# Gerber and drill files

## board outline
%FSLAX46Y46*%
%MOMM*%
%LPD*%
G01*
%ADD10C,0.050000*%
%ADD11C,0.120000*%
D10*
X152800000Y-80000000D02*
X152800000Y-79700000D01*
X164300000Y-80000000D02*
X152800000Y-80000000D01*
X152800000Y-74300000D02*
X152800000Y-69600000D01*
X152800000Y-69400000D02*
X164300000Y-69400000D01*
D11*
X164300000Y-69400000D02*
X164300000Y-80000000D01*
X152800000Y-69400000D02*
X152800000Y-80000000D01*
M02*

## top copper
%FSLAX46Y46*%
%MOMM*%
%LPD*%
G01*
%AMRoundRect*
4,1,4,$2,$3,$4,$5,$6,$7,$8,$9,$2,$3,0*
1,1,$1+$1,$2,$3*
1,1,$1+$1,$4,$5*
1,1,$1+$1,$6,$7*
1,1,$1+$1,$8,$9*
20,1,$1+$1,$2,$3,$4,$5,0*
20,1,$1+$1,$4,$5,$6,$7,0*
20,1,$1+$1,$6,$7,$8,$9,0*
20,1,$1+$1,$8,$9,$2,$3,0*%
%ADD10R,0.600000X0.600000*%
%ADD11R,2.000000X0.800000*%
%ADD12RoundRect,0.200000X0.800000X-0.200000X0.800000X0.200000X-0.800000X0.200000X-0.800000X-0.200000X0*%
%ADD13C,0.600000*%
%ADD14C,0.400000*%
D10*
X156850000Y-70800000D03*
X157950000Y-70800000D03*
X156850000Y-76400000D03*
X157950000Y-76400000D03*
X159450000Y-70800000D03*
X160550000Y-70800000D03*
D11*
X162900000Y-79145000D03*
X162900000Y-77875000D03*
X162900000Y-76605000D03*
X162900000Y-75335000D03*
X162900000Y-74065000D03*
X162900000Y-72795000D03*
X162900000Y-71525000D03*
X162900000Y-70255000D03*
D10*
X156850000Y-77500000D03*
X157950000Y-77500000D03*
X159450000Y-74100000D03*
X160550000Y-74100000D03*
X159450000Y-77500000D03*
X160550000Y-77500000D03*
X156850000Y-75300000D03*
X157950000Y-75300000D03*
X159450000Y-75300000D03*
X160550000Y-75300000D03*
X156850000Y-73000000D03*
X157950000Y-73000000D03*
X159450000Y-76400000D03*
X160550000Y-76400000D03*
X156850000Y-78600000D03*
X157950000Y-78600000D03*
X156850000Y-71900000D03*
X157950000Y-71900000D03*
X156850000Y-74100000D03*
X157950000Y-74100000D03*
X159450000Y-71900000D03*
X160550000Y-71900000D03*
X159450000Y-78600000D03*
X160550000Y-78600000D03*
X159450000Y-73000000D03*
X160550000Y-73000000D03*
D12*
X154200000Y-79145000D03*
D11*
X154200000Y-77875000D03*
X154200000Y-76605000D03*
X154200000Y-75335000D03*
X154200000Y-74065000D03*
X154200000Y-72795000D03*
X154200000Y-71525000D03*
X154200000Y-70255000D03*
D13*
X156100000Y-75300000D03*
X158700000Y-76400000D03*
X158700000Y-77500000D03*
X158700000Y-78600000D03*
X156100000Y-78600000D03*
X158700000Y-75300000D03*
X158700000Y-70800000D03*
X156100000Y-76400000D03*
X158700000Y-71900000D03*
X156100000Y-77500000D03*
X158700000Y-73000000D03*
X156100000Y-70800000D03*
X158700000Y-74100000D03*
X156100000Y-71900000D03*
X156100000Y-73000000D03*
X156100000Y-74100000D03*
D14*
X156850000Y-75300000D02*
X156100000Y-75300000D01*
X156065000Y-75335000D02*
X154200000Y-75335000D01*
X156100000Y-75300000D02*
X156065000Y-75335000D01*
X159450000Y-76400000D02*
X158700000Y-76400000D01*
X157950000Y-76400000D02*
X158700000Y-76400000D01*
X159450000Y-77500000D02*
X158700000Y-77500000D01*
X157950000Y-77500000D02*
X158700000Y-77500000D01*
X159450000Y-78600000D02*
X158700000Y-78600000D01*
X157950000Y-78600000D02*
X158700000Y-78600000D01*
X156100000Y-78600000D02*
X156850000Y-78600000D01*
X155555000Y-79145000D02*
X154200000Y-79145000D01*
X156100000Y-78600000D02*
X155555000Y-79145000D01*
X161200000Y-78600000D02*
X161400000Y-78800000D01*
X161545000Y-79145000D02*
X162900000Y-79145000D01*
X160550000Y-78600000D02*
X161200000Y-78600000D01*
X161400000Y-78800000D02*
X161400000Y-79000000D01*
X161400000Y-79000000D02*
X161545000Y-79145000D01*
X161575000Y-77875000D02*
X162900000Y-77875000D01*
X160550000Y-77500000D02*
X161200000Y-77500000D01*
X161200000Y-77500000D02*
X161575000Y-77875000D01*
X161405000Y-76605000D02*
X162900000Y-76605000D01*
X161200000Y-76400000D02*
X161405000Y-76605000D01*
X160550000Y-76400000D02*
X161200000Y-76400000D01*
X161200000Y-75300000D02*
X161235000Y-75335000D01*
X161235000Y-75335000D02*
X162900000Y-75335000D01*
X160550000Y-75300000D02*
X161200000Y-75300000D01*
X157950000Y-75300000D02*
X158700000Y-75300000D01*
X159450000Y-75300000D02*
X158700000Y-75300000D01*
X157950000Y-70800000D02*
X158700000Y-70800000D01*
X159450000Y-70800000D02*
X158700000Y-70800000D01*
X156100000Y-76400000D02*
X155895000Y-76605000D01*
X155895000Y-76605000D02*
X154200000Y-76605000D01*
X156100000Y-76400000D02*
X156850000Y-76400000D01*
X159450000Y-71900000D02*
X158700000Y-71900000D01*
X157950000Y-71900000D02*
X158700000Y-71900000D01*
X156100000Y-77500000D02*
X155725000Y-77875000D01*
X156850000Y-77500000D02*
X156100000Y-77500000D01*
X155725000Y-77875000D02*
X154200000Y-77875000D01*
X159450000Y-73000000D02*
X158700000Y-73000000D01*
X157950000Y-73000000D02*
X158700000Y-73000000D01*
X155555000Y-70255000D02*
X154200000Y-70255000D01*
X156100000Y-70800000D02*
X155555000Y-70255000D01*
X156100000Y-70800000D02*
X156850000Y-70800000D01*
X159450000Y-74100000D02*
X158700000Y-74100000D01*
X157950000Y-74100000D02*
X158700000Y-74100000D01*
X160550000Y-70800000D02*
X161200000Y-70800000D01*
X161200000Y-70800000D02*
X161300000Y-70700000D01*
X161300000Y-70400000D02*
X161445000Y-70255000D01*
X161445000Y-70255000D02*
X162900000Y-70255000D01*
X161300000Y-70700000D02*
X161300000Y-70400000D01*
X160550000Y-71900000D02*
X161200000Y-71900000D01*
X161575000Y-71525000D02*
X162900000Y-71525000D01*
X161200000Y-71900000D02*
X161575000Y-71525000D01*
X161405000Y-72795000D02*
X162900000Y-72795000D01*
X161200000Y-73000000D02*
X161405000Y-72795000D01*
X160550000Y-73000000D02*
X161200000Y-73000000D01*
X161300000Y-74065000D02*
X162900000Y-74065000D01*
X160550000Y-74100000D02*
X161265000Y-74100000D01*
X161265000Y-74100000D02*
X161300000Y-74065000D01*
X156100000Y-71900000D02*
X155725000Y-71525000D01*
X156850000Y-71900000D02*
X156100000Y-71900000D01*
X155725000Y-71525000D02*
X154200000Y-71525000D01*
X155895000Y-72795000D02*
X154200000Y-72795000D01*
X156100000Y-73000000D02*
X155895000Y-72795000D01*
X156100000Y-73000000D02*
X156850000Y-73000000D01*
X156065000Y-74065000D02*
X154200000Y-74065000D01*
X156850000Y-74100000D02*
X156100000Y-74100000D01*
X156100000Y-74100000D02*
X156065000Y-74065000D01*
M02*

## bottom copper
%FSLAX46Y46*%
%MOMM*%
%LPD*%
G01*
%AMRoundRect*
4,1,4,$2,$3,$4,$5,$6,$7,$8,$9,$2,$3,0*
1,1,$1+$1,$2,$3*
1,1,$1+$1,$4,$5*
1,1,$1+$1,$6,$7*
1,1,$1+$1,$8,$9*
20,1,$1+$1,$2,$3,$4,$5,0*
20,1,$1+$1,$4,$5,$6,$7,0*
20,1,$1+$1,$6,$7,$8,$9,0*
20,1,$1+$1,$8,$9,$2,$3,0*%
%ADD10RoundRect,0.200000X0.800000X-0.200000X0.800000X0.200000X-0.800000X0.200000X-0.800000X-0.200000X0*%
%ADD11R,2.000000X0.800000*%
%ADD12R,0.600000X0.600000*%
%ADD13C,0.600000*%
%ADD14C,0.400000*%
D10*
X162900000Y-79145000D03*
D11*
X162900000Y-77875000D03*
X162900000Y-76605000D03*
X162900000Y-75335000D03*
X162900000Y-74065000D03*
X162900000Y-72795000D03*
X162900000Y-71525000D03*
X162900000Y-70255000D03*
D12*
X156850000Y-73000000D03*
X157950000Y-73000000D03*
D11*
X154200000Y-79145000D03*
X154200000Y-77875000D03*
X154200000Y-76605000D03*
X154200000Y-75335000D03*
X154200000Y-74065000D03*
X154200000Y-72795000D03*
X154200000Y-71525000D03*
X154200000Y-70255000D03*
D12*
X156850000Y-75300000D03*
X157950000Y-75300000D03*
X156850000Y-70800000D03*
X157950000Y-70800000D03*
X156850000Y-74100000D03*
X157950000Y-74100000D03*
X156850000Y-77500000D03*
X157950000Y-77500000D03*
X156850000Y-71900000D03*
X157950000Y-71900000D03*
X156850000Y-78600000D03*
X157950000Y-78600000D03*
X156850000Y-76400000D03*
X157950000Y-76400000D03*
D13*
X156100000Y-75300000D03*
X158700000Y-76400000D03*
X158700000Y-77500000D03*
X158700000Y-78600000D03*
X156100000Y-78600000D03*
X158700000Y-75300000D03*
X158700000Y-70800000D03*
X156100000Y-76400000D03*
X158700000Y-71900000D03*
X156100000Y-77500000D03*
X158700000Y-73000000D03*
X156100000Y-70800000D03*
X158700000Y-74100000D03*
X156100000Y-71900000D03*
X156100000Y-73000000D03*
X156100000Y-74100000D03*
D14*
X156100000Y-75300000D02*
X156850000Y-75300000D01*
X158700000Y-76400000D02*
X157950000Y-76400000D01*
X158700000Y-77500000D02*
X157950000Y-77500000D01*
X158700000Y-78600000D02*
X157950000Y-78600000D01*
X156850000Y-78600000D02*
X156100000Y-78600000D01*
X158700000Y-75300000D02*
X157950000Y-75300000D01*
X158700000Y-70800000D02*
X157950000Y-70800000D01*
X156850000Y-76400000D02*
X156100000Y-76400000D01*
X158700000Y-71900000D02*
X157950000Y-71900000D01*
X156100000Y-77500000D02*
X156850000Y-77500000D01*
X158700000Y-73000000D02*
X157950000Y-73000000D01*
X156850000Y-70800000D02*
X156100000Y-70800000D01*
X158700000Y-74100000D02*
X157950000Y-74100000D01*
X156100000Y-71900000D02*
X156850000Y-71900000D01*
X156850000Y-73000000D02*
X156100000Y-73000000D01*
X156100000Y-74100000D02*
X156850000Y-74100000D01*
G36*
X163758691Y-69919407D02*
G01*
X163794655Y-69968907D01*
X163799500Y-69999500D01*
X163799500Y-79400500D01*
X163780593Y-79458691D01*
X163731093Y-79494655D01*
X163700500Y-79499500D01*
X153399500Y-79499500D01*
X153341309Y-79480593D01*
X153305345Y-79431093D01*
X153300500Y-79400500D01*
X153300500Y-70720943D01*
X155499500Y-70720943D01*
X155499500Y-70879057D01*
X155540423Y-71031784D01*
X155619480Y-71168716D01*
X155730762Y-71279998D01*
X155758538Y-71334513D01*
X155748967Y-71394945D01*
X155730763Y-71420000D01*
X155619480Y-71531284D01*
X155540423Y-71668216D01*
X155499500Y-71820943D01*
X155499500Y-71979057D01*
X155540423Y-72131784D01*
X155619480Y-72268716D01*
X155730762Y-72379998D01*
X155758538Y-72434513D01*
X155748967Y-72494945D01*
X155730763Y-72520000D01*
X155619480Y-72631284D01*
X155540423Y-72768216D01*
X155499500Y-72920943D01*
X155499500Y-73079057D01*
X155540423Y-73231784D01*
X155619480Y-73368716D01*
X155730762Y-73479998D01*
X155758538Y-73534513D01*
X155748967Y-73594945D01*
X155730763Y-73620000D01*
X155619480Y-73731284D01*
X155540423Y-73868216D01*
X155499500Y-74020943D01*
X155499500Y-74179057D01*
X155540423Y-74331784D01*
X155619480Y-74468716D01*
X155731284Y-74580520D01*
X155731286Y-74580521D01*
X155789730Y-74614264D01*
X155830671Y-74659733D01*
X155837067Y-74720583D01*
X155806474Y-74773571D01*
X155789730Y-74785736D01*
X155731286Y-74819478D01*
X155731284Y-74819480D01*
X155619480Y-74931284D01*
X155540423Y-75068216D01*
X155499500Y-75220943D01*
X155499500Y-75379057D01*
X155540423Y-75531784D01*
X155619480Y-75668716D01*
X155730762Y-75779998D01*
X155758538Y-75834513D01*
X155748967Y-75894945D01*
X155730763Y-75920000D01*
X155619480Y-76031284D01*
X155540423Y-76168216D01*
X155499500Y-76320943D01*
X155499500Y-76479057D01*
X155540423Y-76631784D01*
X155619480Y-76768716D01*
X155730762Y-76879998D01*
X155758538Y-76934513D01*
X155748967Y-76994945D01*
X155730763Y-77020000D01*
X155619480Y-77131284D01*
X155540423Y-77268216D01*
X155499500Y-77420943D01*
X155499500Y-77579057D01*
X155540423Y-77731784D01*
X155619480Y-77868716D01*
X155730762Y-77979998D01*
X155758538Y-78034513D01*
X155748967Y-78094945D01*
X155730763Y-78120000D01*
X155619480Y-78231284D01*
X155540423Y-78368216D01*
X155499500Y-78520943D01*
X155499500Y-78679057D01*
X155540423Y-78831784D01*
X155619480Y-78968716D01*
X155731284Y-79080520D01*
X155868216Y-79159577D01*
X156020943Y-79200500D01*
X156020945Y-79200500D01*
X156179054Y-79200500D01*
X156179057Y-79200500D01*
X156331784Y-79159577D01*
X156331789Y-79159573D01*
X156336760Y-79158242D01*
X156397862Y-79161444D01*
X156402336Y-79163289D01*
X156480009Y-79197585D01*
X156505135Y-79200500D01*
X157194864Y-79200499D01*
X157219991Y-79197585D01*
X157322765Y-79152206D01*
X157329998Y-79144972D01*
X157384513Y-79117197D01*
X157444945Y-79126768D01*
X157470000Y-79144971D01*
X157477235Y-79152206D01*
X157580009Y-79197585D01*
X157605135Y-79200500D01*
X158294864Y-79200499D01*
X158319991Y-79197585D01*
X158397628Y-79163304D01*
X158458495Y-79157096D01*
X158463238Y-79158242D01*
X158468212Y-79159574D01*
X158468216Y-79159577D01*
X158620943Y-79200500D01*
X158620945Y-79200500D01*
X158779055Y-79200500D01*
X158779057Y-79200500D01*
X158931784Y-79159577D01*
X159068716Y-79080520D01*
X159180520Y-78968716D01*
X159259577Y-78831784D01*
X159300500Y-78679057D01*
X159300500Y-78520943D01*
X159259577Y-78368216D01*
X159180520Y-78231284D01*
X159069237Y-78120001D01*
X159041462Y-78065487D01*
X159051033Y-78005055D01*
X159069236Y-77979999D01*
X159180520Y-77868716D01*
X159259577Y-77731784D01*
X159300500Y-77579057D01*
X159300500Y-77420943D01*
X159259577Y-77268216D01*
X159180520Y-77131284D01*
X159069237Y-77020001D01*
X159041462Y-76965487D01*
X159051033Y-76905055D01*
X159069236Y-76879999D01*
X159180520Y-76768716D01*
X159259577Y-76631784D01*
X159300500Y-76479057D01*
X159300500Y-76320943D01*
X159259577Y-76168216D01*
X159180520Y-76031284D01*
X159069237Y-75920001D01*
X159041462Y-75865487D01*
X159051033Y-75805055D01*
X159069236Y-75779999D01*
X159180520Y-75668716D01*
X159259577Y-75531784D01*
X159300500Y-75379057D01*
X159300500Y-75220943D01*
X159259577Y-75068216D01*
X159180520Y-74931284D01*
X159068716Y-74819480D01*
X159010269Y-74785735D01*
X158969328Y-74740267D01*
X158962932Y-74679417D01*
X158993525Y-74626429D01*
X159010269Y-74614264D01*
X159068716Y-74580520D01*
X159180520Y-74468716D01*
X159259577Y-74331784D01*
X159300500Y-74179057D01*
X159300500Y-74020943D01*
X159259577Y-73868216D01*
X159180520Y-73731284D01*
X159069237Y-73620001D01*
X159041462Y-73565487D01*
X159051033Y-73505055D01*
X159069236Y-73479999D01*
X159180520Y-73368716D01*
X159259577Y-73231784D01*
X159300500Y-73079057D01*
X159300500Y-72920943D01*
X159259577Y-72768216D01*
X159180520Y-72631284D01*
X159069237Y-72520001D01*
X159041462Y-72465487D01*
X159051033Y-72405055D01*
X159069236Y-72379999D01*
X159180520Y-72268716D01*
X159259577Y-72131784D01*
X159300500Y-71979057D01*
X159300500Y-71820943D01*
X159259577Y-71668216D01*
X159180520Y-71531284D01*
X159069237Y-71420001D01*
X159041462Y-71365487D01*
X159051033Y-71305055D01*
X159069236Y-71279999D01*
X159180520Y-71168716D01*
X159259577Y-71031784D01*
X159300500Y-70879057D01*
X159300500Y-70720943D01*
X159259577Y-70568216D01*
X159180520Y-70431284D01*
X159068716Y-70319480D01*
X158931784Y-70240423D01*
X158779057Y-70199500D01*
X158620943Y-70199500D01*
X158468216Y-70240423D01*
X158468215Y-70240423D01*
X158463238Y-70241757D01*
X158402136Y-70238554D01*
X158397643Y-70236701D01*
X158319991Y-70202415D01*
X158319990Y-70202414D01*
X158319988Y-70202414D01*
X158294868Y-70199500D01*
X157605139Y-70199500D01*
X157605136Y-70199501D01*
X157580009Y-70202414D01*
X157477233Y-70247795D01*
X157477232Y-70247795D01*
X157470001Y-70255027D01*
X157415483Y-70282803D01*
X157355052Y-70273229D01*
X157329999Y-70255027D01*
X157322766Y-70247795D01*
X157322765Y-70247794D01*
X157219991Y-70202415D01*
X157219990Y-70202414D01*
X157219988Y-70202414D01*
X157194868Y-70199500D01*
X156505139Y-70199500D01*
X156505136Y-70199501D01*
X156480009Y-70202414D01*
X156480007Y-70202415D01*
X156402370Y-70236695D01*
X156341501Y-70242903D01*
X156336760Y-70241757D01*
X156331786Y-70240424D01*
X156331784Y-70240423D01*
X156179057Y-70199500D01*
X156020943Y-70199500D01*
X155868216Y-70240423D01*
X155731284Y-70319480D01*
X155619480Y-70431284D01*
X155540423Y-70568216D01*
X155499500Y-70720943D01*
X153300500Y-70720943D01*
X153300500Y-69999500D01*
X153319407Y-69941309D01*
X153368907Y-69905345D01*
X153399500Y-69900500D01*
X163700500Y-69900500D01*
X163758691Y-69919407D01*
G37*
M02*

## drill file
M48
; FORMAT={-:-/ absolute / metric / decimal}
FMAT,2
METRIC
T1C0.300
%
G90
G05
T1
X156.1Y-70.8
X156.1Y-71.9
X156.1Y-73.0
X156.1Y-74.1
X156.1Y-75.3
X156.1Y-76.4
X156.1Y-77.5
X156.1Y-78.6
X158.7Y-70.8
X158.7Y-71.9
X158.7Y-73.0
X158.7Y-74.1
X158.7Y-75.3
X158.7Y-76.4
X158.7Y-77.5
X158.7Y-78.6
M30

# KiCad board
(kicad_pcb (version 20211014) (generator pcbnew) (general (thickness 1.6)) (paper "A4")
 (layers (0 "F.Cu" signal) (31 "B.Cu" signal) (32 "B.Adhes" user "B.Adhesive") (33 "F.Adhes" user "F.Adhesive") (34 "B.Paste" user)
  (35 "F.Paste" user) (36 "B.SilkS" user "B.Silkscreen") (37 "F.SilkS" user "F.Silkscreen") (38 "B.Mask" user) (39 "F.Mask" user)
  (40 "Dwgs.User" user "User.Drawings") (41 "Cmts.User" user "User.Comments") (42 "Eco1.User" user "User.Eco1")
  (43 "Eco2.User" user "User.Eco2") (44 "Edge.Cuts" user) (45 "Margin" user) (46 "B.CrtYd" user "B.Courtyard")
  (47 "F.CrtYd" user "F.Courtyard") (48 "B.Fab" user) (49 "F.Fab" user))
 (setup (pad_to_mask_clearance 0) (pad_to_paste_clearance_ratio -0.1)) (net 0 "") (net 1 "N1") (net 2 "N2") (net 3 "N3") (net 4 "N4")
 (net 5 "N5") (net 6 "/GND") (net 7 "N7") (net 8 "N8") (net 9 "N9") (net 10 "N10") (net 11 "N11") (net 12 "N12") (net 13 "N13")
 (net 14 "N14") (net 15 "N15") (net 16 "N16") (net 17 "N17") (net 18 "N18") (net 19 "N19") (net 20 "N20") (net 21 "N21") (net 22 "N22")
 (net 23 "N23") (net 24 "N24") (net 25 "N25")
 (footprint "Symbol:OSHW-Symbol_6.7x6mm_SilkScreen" (layer "F.Cu") (at 147 76.2)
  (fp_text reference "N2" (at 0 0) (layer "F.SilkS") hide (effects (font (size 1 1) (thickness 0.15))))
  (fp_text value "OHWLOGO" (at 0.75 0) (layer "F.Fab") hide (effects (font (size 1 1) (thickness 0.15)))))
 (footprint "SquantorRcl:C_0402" (layer "F.Cu") (at 157.4 70.8)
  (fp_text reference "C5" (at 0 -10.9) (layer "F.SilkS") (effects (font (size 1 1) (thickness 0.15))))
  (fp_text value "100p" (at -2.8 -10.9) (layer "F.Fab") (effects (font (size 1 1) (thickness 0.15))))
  (pad "1" smd rect (at -0.55 0) (size 0.6 0.6) (layers "F.Cu" "F.Paste" "F.Mask") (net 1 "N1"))
  (pad "2" smd rect (at 0.55 0) (size 0.6 0.6) (layers "F.Cu" "F.Paste" "F.Mask") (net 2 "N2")))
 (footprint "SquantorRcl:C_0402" (layer "F.Cu") (at 157.4 76.4)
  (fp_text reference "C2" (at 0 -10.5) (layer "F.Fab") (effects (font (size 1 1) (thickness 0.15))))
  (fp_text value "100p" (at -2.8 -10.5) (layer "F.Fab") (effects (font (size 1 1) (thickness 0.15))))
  (pad "1" smd rect (at -0.55 0) (size 0.6 0.6) (layers "F.Cu" "F.Paste" "F.Mask") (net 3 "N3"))
  (pad "2" smd rect (at 0.55 0) (size 0.6 0.6) (layers "F.Cu" "F.Paste" "F.Mask") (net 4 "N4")))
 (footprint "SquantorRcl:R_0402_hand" (layer "F.Cu") (at 160 70.8)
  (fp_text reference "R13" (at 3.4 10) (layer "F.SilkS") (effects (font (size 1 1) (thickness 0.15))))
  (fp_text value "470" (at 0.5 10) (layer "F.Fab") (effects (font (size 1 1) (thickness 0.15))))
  (pad "1" smd rect (at -0.55 0) (size 0.6 0.6) (layers "F.Cu" "F.Paste" "F.Mask") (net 2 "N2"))
  (pad "2" smd rect (at 0.55 0) (size 0.6 0.6) (layers "F.Cu" "F.Paste" "F.Mask") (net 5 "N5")))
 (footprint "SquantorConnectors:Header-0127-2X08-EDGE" (layer "F.Cu") (at 161.8 74.7 90)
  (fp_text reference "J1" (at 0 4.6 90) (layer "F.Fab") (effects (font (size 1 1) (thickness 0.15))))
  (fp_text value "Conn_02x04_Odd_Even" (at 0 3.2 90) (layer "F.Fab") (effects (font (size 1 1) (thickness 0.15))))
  (fp_line (start 5.3 2.5) (end -5.3 2.5) (layer "Edge.Cuts") (width 0.12))
  (pad "1" smd roundrect (at -4.445 1.1 90) (size 0.8 2) (layers "B.Cu" "B.Paste" "B.Mask") (roundrect_rratio 0.25) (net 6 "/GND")
   (zone_connect 2))
  (pad "2" smd rect (at -4.445 1.1 90) (size 0.8 2) (layers "F.Cu" "F.Paste" "F.Mask") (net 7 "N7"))
  (pad "3" smd rect (at -3.175 1.1 90) (size 0.8 2) (layers "B.Cu" "B.Paste" "B.Mask") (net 6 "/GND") (zone_connect 2))
  (pad "4" smd rect (at -3.175 1.1 90) (size 0.8 2) (layers "F.Cu" "F.Paste" "F.Mask") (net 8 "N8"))
  (pad "5" smd rect (at -1.905 1.1 90) (size 0.8 2) (layers "B.Cu" "B.Paste" "B.Mask") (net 6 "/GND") (zone_connect 2))
  (pad "6" smd rect (at -1.905 1.1 90) (size 0.8 2) (layers "F.Cu" "F.Paste" "F.Mask") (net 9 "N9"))
  (pad "7" smd rect (at -0.635 1.1 90) (size 0.8 2) (layers "B.Cu" "B.Paste" "B.Mask") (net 6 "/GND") (zone_connect 2))
  (pad "8" smd rect (at -0.635 1.1 90) (size 0.8 2) (layers "F.Cu" "F.Paste" "F.Mask") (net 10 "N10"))
  (pad "9" smd rect (at 0.635 1.1 90) (size 0.8 2) (layers "B.Cu" "B.Paste" "B.Mask") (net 6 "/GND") (zone_connect 2))
  (pad "10" smd rect (at 0.635 1.1 90) (size 0.8 2) (layers "F.Cu" "F.Paste" "F.Mask") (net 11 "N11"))
  (pad "11" smd rect (at 1.905 1.1 90) (size 0.8 2) (layers "B.Cu" "B.Paste" "B.Mask") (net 6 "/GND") (zone_connect 2))
  (pad "12" smd rect (at 1.905 1.1 90) (size 0.8 2) (layers "F.Cu" "F.Paste" "F.Mask") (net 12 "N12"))
  (pad "13" smd rect (at 3.175 1.1 90) (size 0.8 2) (layers "B.Cu" "B.Paste" "B.Mask") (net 6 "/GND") (zone_connect 2))
  (pad "14" smd rect (at 3.175 1.1 90) (size 0.8 2) (layers "F.Cu" "F.Paste" "F.Mask") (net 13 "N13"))
  (pad "15" smd rect (at 4.445 1.1 90) (size 0.8 2) (layers "B.Cu" "B.Paste" "B.Mask") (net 6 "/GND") (zone_connect 2))
  (pad "16" smd rect (at 4.445 1.1 90) (size 0.8 2) (layers "F.Cu" "F.Paste" "F.Mask") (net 5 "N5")))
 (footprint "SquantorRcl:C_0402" (layer "F.Cu") (at 157.4 77.5)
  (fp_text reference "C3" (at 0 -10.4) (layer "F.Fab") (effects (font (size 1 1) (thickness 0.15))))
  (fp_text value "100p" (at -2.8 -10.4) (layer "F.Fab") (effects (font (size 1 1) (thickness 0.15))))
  (pad "1" smd rect (at -0.55 0) (size 0.6 0.6) (layers "F.Cu" "F.Paste" "F.Mask") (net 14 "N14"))
  (pad "2" smd rect (at 0.55 0) (size 0.6 0.6) (layers "F.Cu" "F.Paste" "F.Mask") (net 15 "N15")))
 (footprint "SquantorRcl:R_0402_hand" (layer "F.Cu") (at 160 74.1)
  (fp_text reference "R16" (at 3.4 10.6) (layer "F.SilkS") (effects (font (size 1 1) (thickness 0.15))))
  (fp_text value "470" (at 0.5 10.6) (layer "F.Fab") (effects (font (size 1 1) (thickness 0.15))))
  (pad "1" smd rect (at -0.55 0) (size 0.6 0.6) (layers "F.Cu" "F.Paste" "F.Mask") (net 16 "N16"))
  (pad "2" smd rect (at 0.55 0) (size 0.6 0.6) (layers "F.Cu" "F.Paste" "F.Mask") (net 11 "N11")))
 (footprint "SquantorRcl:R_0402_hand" (layer "F.Cu") (at 160 77.5)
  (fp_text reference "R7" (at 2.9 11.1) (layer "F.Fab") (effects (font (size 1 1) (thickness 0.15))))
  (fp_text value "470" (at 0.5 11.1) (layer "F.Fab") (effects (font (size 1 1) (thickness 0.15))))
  (pad "1" smd rect (at -0.55 0) (size 0.6 0.6) (layers "F.Cu" "F.Paste" "F.Mask") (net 15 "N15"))
  (pad "2" smd rect (at 0.55 0) (size 0.6 0.6) (layers "F.Cu" "F.Paste" "F.Mask") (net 8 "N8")))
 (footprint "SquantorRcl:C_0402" (layer "F.Cu") (at 157.4 75.3)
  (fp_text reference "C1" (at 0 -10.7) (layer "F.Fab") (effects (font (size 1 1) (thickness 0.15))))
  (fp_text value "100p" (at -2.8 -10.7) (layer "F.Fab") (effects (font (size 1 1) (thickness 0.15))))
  (pad "1" smd rect (at -0.55 0) (size 0.6 0.6) (layers "F.Cu" "F.Paste" "F.Mask") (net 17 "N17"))
  (pad "2" smd rect (at 0.55 0) (size 0.6 0.6) (layers "F.Cu" "F.Paste" "F.Mask") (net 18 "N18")))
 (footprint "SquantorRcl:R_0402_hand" (layer "F.Cu") (at 160 75.3)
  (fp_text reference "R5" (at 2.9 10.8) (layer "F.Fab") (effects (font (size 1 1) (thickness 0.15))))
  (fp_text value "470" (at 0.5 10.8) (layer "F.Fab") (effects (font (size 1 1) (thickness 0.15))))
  (pad "1" smd rect (at -0.55 0) (size 0.6 0.6) (layers "F.Cu" "F.Paste" "F.Mask") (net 18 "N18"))
  (pad "2" smd rect (at 0.55 0) (size 0.6 0.6) (layers "F.Cu" "F.Paste" "F.Mask") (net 10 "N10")))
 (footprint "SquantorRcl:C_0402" (layer "F.Cu") (at 157.4 73)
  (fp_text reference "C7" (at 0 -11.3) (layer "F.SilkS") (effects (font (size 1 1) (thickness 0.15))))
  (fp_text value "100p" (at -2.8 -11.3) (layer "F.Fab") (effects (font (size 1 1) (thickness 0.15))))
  (pad "1" smd rect (at -0.55 0) (size 0.6 0.6) (layers "F.Cu" "F.Paste" "F.Mask") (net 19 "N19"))
  (pad "2" smd rect (at 0.55 0) (size 0.6 0.6) (layers "F.Cu" "F.Paste" "F.Mask") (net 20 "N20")))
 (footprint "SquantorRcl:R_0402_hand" (layer "F.Cu") (at 160 76.4)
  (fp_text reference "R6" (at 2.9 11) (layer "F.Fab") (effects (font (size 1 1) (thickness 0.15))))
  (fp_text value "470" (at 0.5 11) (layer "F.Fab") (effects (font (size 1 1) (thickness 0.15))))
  (pad "1" smd rect (at -0.55 0) (size 0.6 0.6) (layers "F.Cu" "F.Paste" "F.Mask") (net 4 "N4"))
  (pad "2" smd rect (at 0.55 0) (size 0.6 0.6) (layers "F.Cu" "F.Paste" "F.Mask") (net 9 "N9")))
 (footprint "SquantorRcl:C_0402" (layer "F.Cu") (at 157.4 78.6)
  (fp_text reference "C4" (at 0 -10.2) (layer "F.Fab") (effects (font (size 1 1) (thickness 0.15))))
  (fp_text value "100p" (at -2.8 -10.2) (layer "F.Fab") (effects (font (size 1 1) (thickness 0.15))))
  (pad "1" smd rect (at -0.55 0) (size 0.6 0.6) (layers "F.Cu" "F.Paste" "F.Mask") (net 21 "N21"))
  (pad "2" smd rect (at 0.55 0) (size 0.6 0.6) (layers "F.Cu" "F.Paste" "F.Mask") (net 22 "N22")))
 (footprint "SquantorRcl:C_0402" (layer "F.Cu") (at 157.4 71.9)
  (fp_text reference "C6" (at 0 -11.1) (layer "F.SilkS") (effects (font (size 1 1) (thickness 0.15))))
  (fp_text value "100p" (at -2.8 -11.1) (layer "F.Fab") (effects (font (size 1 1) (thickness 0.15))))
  (pad "1" smd rect (at -0.55 0) (size 0.6 0.6) (layers "F.Cu" "F.Paste" "F.Mask") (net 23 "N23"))
  (pad "2" smd rect (at 0.55 0) (size 0.6 0.6) (layers "F.Cu" "F.Paste" "F.Mask") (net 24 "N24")))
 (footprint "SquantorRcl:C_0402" (layer "F.Cu") (at 157.4 74.1)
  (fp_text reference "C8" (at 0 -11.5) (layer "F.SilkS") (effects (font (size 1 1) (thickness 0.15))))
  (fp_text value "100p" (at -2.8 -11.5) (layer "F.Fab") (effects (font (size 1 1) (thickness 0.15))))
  (pad "1" smd rect (at -0.55 0) (size 0.6 0.6) (layers "F.Cu" "F.Paste" "F.Mask") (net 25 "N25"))
  (pad "2" smd rect (at 0.55 0) (size 0.6 0.6) (layers "F.Cu" "F.Paste" "F.Mask") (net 16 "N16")))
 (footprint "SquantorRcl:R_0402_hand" (layer "F.Cu") (at 160 71.9)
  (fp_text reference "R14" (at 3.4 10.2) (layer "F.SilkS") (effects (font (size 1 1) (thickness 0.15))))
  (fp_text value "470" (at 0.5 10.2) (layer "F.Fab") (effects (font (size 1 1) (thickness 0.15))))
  (pad "1" smd rect (at -0.55 0) (size 0.6 0.6) (layers "F.Cu" "F.Paste" "F.Mask") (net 24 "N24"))
  (pad "2" smd rect (at 0.55 0) (size 0.6 0.6) (layers "F.Cu" "F.Paste" "F.Mask") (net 13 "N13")))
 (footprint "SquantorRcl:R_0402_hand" (layer "F.Cu") (at 160 78.6)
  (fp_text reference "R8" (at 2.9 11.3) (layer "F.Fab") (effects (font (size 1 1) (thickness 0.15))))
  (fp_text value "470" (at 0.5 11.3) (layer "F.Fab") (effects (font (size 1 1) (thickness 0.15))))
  (pad "1" smd rect (at -0.55 0) (size 0.6 0.6) (layers "F.Cu" "F.Paste" "F.Mask") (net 22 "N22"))
  (pad "2" smd rect (at 0.55 0) (size 0.6 0.6) (layers "F.Cu" "F.Paste" "F.Mask") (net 7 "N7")))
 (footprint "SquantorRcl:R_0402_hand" (layer "F.Cu") (at 160 73)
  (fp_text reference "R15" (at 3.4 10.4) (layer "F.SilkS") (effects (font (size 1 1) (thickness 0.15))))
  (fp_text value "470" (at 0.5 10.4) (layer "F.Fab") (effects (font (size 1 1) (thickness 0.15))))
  (pad "1" smd rect (at -0.55 0) (size 0.6 0.6) (layers "F.Cu" "F.Paste" "F.Mask") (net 20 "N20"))
  (pad "2" smd rect (at 0.55 0) (size 0.6 0.6) (layers "F.Cu" "F.Paste" "F.Mask") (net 12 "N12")))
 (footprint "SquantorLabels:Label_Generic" (layer "B.Cu") (at 159.7875 74.4 -90)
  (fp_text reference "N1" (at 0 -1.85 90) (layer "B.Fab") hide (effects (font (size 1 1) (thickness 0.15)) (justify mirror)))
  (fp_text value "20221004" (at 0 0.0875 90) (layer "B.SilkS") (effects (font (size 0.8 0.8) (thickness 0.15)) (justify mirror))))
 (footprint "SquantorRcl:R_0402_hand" (layer "B.Cu") (at 157.4 73)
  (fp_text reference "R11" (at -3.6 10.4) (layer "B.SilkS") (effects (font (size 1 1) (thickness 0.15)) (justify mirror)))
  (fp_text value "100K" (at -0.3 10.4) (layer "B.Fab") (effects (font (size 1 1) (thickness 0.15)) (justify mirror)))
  (pad "1" smd rect (at -0.55 0) (size 0.6 0.6) (layers "B.Cu" "B.Paste" "B.Mask") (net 19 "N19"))
  (pad "2" smd rect (at 0.55 0) (size 0.6 0.6) (layers "B.Cu" "B.Paste" "B.Mask") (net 20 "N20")))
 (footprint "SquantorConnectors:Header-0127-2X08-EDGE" (layer "B.Cu") (at 155.3 74.7 90)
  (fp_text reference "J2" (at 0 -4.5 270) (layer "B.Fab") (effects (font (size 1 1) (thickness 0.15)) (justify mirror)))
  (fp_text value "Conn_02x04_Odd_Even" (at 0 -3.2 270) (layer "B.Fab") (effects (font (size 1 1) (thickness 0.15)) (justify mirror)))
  (fp_line (start 5.3 -2.5) (end -5.3 -2.5) (layer "Edge.Cuts") (width 0.12))
  (pad "1" smd roundrect (at -4.445 -1.1 90) (size 0.8 2) (layers "F.Cu" "F.Paste" "F.Mask") (roundrect_rratio 0.25) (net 21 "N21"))
  (pad "2" smd rect (at -4.445 -1.1 90) (size 0.8 2) (layers "B.Cu" "B.Paste" "B.Mask") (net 6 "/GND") (zone_connect 2))
  (pad "3" smd rect (at -3.175 -1.1 90) (size 0.8 2) (layers "F.Cu" "F.Paste" "F.Mask") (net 14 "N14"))
  (pad "4" smd rect (at -3.175 -1.1 90) (size 0.8 2) (layers "B.Cu" "B.Paste" "B.Mask") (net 6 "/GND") (zone_connect 2))
  (pad "5" smd rect (at -1.905 -1.1 90) (size 0.8 2) (layers "F.Cu" "F.Paste" "F.Mask") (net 3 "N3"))
  (pad "6" smd rect (at -1.905 -1.1 90) (size 0.8 2) (layers "B.Cu" "B.Paste" "B.Mask") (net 6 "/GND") (zone_connect 2))
  (pad "7" smd rect (at -0.635 -1.1 90) (size 0.8 2) (layers "F.Cu" "F.Paste" "F.Mask") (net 17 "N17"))
  (pad "8" smd rect (at -0.635 -1.1 90) (size 0.8 2) (layers "B.Cu" "B.Paste" "B.Mask") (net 6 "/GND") (zone_connect 2))
  (pad "9" smd rect (at 0.635 -1.1 90) (size 0.8 2) (layers "F.Cu" "F.Paste" "F.Mask") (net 25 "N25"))
  (pad "10" smd rect (at 0.635 -1.1 90) (size 0.8 2) (layers "B.Cu" "B.Paste" "B.Mask") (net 6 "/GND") (zone_connect 2))
  (pad "11" smd rect (at 1.905 -1.1 90) (size 0.8 2) (layers "F.Cu" "F.Paste" "F.Mask") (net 19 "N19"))
  (pad "12" smd rect (at 1.905 -1.1 90) (size 0.8 2) (layers "B.Cu" "B.Paste" "B.Mask") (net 6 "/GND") (zone_connect 2))
  (pad "13" smd rect (at 3.175 -1.1 90) (size 0.8 2) (layers "F.Cu" "F.Paste" "F.Mask") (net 23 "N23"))
  (pad "14" smd rect (at 3.175 -1.1 90) (size 0.8 2) (layers "B.Cu" "B.Paste" "B.Mask") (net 6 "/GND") (zone_connect 2))
  (pad "15" smd rect (at 4.445 -1.1 90) (size 0.8 2) (layers "F.Cu" "F.Paste" "F.Mask") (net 1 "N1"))
  (pad "16" smd rect (at 4.445 -1.1 90) (size 0.8 2) (layers "B.Cu" "B.Paste" "B.Mask") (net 6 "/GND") (zone_connect 2)))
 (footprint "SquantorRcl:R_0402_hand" (layer "B.Cu") (at 157.4 75.3)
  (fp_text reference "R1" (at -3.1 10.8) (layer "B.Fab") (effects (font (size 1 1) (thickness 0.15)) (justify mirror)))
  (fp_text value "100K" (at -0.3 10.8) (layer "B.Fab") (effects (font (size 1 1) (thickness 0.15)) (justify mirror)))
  (pad "1" smd rect (at -0.55 0) (size 0.6 0.6) (layers "B.Cu" "B.Paste" "B.Mask") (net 17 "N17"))
  (pad "2" smd rect (at 0.55 0) (size 0.6 0.6) (layers "B.Cu" "B.Paste" "B.Mask") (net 18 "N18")))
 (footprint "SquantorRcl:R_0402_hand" (layer "B.Cu") (at 157.4 70.8)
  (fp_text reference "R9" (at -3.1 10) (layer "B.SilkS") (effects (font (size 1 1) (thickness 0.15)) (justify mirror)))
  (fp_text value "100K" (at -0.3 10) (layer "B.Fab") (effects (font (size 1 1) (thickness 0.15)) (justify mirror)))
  (pad "1" smd rect (at -0.55 0) (size 0.6 0.6) (layers "B.Cu" "B.Paste" "B.Mask") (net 1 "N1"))
  (pad "2" smd rect (at 0.55 0) (size 0.6 0.6) (layers "B.Cu" "B.Paste" "B.Mask") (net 2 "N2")))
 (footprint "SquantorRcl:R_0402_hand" (layer "B.Cu") (at 157.4 74.1)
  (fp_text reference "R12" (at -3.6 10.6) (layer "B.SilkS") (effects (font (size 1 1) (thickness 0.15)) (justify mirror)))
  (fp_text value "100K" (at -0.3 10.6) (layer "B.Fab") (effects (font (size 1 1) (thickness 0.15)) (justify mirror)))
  (pad "1" smd rect (at -0.55 0) (size 0.6 0.6) (layers "B.Cu" "B.Paste" "B.Mask") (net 25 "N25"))
  (pad "2" smd rect (at 0.55 0) (size 0.6 0.6) (layers "B.Cu" "B.Paste" "B.Mask") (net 16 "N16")))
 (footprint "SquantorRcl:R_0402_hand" (layer "B.Cu") (at 157.4 77.5)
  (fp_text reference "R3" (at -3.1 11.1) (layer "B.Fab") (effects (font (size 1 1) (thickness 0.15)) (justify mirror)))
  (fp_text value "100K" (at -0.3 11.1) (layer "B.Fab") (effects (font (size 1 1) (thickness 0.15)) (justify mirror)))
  (pad "1" smd rect (at -0.55 0) (size 0.6 0.6) (layers "B.Cu" "B.Paste" "B.Mask") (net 14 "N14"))
  (pad "2" smd rect (at 0.55 0) (size 0.6 0.6) (layers "B.Cu" "B.Paste" "B.Mask") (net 15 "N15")))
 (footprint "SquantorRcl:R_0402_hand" (layer "B.Cu") (at 157.4 71.9)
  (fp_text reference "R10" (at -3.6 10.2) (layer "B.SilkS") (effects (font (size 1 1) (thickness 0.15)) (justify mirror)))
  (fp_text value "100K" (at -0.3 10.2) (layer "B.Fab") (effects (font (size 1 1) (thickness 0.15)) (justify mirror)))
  (pad "1" smd rect (at -0.55 0) (size 0.6 0.6) (layers "B.Cu" "B.Paste" "B.Mask") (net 23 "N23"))
  (pad "2" smd rect (at 0.55 0) (size 0.6 0.6) (layers "B.Cu" "B.Paste" "B.Mask") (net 24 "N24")))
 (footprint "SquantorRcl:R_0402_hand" (layer "B.Cu") (at 157.4 78.6)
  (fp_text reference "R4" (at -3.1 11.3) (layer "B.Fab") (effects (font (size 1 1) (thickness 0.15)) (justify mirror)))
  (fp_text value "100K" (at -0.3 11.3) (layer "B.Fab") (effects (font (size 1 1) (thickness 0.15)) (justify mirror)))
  (pad "1" smd rect (at -0.55 0) (size 0.6 0.6) (layers "B.Cu" "B.Paste" "B.Mask") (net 21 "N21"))
  (pad "2" smd rect (at 0.55 0) (size 0.6 0.6) (layers "B.Cu" "B.Paste" "B.Mask") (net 22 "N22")))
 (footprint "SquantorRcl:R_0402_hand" (layer "B.Cu") (at 157.4 76.4)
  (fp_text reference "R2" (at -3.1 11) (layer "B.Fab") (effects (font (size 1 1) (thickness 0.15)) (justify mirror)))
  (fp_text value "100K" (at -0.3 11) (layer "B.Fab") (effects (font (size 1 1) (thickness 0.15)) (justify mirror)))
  (pad "1" smd rect (at -0.55 0) (size 0.6 0.6) (layers "B.Cu" "B.Paste" "B.Mask") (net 3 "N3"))
  (pad "2" smd rect (at 0.55 0) (size 0.6 0.6) (layers "B.Cu" "B.Paste" "B.Mask") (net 4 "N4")))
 (gr_line (start 152.8 80) (end 152.8 79.7) (layer "Edge.Cuts") (width 0.05))
 (gr_line (start 164.3 80) (end 152.8 80) (layer "Edge.Cuts") (width 0.05))
 (gr_line (start 152.8 74.3) (end 152.8 69.6) (layer "Edge.Cuts") (width 0.05))
 (gr_line (start 152.8 69.4) (end 164.3 69.4) (layer "Edge.Cuts") (width 0.05))
 (segment (start 156.85 75.3) (end 156.1 75.3) (width 0.4) (layer "F.Cu") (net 17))
 (segment (start 156.065 75.335) (end 154.2 75.335) (width 0.4) (layer "F.Cu") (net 17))
 (segment (start 156.1 75.3) (end 156.065 75.335) (width 0.4) (layer "F.Cu") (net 17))
 (via (at 156.1 75.3) (size 0.6) (drill 0.3) (layers "F.Cu" "B.Cu") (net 17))
 (segment (start 156.1 75.3) (end 156.85 75.3) (width 0.4) (layer "B.Cu") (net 17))
 (segment (start 159.45 76.4) (end 158.7 76.4) (width 0.4) (layer "F.Cu") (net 4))
 (segment (start 157.95 76.4) (end 158.7 76.4) (width 0.4) (layer "F.Cu") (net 4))
 (via (at 158.7 76.4) (size 0.6) (drill 0.3) (layers "F.Cu" "B.Cu") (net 4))
 (segment (start 158.7 76.4) (end 157.95 76.4) (width 0.4) (layer "B.Cu") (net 4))
 (segment (start 159.45 77.5) (end 158.7 77.5) (width 0.4) (layer "F.Cu") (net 15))
 (segment (start 157.95 77.5) (end 158.7 77.5) (width 0.4) (layer "F.Cu") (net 15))
 (via (at 158.7 77.5) (size 0.6) (drill 0.3) (layers "F.Cu" "B.Cu") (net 15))
 (segment (start 158.7 77.5) (end 157.95 77.5) (width 0.4) (layer "B.Cu") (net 15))
 (segment (start 159.45 78.6) (end 158.7 78.6) (width 0.4) (layer "F.Cu") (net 22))
 (segment (start 157.95 78.6) (end 158.7 78.6) (width 0.4) (layer "F.Cu") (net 22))
 (via (at 158.7 78.6) (size 0.6) (drill 0.3) (layers "F.Cu" "B.Cu") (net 22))
 (segment (start 158.7 78.6) (end 157.95 78.6) (width 0.4) (layer "B.Cu") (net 22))
 (segment (start 156.1 78.6) (end 156.85 78.6) (width 0.4) (layer "F.Cu") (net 21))
 (segment (start 155.555 79.145) (end 154.2 79.145) (width 0.4) (layer "F.Cu") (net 21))
 (segment (start 156.1 78.6) (end 155.555 79.145) (width 0.4) (layer "F.Cu") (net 21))
 (via (at 156.1 78.6) (size 0.6) (drill 0.3) (layers "F.Cu" "B.Cu") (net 21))
 (segment (start 156.85 78.6) (end 156.1 78.6) (width 0.4) (layer "B.Cu") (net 21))
 (segment (start 161.2 78.6) (end 161.4 78.8) (width 0.4) (layer "F.Cu") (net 7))
 (segment (start 161.545 79.145) (end 162.9 79.145) (width 0.4) (layer "F.Cu") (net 7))
 (segment (start 160.55 78.6) (end 161.2 78.6) (width 0.4) (layer "F.Cu") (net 7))
 (segment (start 161.4 78.8) (end 161.4 79) (width 0.4) (layer "F.Cu") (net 7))
 (segment (start 161.4 79) (end 161.545 79.145) (width 0.4) (layer "F.Cu") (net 7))
 (segment (start 161.575 77.875) (end 162.9 77.875) (width 0.4) (layer "F.Cu") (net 8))
 (segment (start 160.55 77.5) (end 161.2 77.5) (width 0.4) (layer "F.Cu") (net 8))
 (segment (start 161.2 77.5) (end 161.575 77.875) (width 0.4) (layer "F.Cu") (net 8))
 (segment (start 161.405 76.605) (end 162.9 76.605) (width 0.4) (layer "F.Cu") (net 9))
 (segment (start 161.2 76.4) (end 161.405 76.605) (width 0.4) (layer "F.Cu") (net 9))
 (segment (start 160.55 76.4) (end 161.2 76.4) (width 0.4) (layer "F.Cu") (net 9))
 (segment (start 161.2 75.3) (end 161.235 75.335) (width 0.4) (layer "F.Cu") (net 10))
 (segment (start 161.235 75.335) (end 162.9 75.335) (width 0.4) (layer "F.Cu") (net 10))
 (segment (start 160.55 75.3) (end 161.2 75.3) (width 0.4) (layer "F.Cu") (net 10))
 (segment (start 157.95 75.3) (end 158.7 75.3) (width 0.4) (layer "F.Cu") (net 18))
 (segment (start 159.45 75.3) (end 158.7 75.3) (width 0.4) (layer "F.Cu") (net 18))
 (via (at 158.7 75.3) (size 0.6) (drill 0.3) (layers "F.Cu" "B.Cu") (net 18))
 (segment (start 158.7 75.3) (end 157.95 75.3) (width 0.4) (layer "B.Cu") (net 18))
 (segment (start 157.95 70.8) (end 158.7 70.8) (width 0.4) (layer "F.Cu") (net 2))
 (segment (start 159.45 70.8) (end 158.7 70.8) (width 0.4) (layer "F.Cu") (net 2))
 (via (at 158.7 70.8) (size 0.6) (drill 0.3) (layers "F.Cu" "B.Cu") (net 2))
 (segment (start 158.7 70.8) (end 157.95 70.8) (width 0.4) (layer "B.Cu") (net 2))
 (segment (start 156.1 76.4) (end 155.895 76.605) (width 0.4) (layer "F.Cu") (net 3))
 (segment (start 155.895 76.605) (end 154.2 76.605) (width 0.4) (layer "F.Cu") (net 3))
 (segment (start 156.1 76.4) (end 156.85 76.4) (width 0.4) (layer "F.Cu") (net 3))
 (via (at 156.1 76.4) (size 0.6) (drill 0.3) (layers "F.Cu" "B.Cu") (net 3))
 (segment (start 156.85 76.4) (end 156.1 76.4) (width 0.4) (layer "B.Cu") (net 3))
 (segment (start 159.45 71.9) (end 158.7 71.9) (width 0.4) (layer "F.Cu") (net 24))
 (segment (start 157.95 71.9) (end 158.7 71.9) (width 0.4) (layer "F.Cu") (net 24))
 (via (at 158.7 71.9) (size 0.6) (drill 0.3) (layers "F.Cu" "B.Cu") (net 24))
 (segment (start 158.7 71.9) (end 157.95 71.9) (width 0.4) (layer "B.Cu") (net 24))
 (segment (start 156.1 77.5) (end 155.725 77.875) (width 0.4) (layer "F.Cu") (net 14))
 (segment (start 156.85 77.5) (end 156.1 77.5) (width 0.4) (layer "F.Cu") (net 14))
 (segment (start 155.725 77.875) (end 154.2 77.875) (width 0.4) (layer "F.Cu") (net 14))
 (via (at 156.1 77.5) (size 0.6) (drill 0.3) (layers "F.Cu" "B.Cu") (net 14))
 (segment (start 156.1 77.5) (end 156.85 77.5) (width 0.4) (layer "B.Cu") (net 14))
 (segment (start 159.45 73) (end 158.7 73) (width 0.4) (layer "F.Cu") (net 20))
 (segment (start 157.95 73) (end 158.7 73) (width 0.4) (layer "F.Cu") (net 20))
 (via (at 158.7 73) (size 0.6) (drill 0.3) (layers "F.Cu" "B.Cu") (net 20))
 (segment (start 158.7 73) (end 157.95 73) (width 0.4) (layer "B.Cu") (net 20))
 (segment (start 155.555 70.255) (end 154.2 70.255) (width 0.4) (layer "F.Cu") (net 1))
 (segment (start 156.1 70.8) (end 155.555 70.255) (width 0.4) (layer "F.Cu") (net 1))
 (segment (start 156.1 70.8) (end 156.85 70.8) (width 0.4) (layer "F.Cu") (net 1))
 (via (at 156.1 70.8) (size 0.6) (drill 0.3) (layers "F.Cu" "B.Cu") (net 1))
 (segment (start 156.85 70.8) (end 156.1 70.8) (width 0.4) (layer "B.Cu") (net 1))
 (segment (start 159.45 74.1) (end 158.7 74.1) (width 0.4) (layer "F.Cu") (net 16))
 (segment (start 157.95 74.1) (end 158.7 74.1) (width 0.4) (layer "F.Cu") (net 16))
 (via (at 158.7 74.1) (size 0.6) (drill 0.3) (layers "F.Cu" "B.Cu") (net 16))
 (segment (start 158.7 74.1) (end 157.95 74.1) (width 0.4) (layer "B.Cu") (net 16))
 (segment (start 160.55 70.8) (end 161.2 70.8) (width 0.4) (layer "F.Cu") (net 5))
 (segment (start 161.2 70.8) (end 161.3 70.7) (width 0.4) (layer "F.Cu") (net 5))
 (segment (start 161.3 70.4) (end 161.445 70.255) (width 0.4) (layer "F.Cu") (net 5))
 (segment (start 161.445 70.255) (end 162.9 70.255) (width 0.4) (layer "F.Cu") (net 5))
 (segment (start 161.3 70.7) (end 161.3 70.4) (width 0.4) (layer "F.Cu") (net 5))
 (segment (start 160.55 71.9) (end 161.2 71.9) (width 0.4) (layer "F.Cu") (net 13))
 (segment (start 161.575 71.525) (end 162.9 71.525) (width 0.4) (layer "F.Cu") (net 13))
 (segment (start 161.2 71.9) (end 161.575 71.525) (width 0.4) (layer "F.Cu") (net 13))
 (segment (start 161.405 72.795) (end 162.9 72.795) (width 0.4) (layer "F.Cu") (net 12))
 (segment (start 161.2 73) (end 161.405 72.795) (width 0.4) (layer "F.Cu") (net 12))
 (segment (start 160.55 73) (end 161.2 73) (width 0.4) (layer "F.Cu") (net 12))
 (segment (start 161.3 74.065) (end 162.9 74.065) (width 0.4) (layer "F.Cu") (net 11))
 (segment (start 160.55 74.1) (end 161.265 74.1) (width 0.4) (layer "F.Cu") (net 11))
 (segment (start 161.265 74.1) (end 161.3 74.065) (width 0.4) (layer "F.Cu") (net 11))
 (segment (start 156.1 71.9) (end 155.725 71.525) (width 0.4) (layer "F.Cu") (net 23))
 (segment (start 156.85 71.9) (end 156.1 71.9) (width 0.4) (layer "F.Cu") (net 23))
 (segment (start 155.725 71.525) (end 154.2 71.525) (width 0.4) (layer "F.Cu") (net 23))
 (via (at 156.1 71.9) (size 0.6) (drill 0.3) (layers "F.Cu" "B.Cu") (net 23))
 (segment (start 156.1 71.9) (end 156.85 71.9) (width 0.4) (layer "B.Cu") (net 23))
 (segment (start 155.895 72.795) (end 154.2 72.795) (width 0.4) (layer "F.Cu") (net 19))
 (segment (start 156.1 73) (end 155.895 72.795) (width 0.4) (layer "F.Cu") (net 19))
 (segment (start 156.1 73) (end 156.85 73) (width 0.4) (layer "F.Cu") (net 19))
 (via (at 156.1 73) (size 0.6) (drill 0.3) (layers "F.Cu" "B.Cu") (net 19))
 (segment (start 156.85 73) (end 156.1 73) (width 0.4) (layer "B.Cu") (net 19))
 (segment (start 156.065 74.065) (end 154.2 74.065) (width 0.4) (layer "F.Cu") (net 25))
 (segment (start 156.85 74.1) (end 156.1 74.1) (width 0.4) (layer "F.Cu") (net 25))
 (segment (start 156.1 74.1) (end 156.065 74.065) (width 0.4) (layer "F.Cu") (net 25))
 (via (at 156.1 74.1) (size 0.6) (drill 0.3) (layers "F.Cu" "B.Cu") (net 25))
 (segment (start 156.1 74.1) (end 156.85 74.1) (width 0.4) (layer "B.Cu") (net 25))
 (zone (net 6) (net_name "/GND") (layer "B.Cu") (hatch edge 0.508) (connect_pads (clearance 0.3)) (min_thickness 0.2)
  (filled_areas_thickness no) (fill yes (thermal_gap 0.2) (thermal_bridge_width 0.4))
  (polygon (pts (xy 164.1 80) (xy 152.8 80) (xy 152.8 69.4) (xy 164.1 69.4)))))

